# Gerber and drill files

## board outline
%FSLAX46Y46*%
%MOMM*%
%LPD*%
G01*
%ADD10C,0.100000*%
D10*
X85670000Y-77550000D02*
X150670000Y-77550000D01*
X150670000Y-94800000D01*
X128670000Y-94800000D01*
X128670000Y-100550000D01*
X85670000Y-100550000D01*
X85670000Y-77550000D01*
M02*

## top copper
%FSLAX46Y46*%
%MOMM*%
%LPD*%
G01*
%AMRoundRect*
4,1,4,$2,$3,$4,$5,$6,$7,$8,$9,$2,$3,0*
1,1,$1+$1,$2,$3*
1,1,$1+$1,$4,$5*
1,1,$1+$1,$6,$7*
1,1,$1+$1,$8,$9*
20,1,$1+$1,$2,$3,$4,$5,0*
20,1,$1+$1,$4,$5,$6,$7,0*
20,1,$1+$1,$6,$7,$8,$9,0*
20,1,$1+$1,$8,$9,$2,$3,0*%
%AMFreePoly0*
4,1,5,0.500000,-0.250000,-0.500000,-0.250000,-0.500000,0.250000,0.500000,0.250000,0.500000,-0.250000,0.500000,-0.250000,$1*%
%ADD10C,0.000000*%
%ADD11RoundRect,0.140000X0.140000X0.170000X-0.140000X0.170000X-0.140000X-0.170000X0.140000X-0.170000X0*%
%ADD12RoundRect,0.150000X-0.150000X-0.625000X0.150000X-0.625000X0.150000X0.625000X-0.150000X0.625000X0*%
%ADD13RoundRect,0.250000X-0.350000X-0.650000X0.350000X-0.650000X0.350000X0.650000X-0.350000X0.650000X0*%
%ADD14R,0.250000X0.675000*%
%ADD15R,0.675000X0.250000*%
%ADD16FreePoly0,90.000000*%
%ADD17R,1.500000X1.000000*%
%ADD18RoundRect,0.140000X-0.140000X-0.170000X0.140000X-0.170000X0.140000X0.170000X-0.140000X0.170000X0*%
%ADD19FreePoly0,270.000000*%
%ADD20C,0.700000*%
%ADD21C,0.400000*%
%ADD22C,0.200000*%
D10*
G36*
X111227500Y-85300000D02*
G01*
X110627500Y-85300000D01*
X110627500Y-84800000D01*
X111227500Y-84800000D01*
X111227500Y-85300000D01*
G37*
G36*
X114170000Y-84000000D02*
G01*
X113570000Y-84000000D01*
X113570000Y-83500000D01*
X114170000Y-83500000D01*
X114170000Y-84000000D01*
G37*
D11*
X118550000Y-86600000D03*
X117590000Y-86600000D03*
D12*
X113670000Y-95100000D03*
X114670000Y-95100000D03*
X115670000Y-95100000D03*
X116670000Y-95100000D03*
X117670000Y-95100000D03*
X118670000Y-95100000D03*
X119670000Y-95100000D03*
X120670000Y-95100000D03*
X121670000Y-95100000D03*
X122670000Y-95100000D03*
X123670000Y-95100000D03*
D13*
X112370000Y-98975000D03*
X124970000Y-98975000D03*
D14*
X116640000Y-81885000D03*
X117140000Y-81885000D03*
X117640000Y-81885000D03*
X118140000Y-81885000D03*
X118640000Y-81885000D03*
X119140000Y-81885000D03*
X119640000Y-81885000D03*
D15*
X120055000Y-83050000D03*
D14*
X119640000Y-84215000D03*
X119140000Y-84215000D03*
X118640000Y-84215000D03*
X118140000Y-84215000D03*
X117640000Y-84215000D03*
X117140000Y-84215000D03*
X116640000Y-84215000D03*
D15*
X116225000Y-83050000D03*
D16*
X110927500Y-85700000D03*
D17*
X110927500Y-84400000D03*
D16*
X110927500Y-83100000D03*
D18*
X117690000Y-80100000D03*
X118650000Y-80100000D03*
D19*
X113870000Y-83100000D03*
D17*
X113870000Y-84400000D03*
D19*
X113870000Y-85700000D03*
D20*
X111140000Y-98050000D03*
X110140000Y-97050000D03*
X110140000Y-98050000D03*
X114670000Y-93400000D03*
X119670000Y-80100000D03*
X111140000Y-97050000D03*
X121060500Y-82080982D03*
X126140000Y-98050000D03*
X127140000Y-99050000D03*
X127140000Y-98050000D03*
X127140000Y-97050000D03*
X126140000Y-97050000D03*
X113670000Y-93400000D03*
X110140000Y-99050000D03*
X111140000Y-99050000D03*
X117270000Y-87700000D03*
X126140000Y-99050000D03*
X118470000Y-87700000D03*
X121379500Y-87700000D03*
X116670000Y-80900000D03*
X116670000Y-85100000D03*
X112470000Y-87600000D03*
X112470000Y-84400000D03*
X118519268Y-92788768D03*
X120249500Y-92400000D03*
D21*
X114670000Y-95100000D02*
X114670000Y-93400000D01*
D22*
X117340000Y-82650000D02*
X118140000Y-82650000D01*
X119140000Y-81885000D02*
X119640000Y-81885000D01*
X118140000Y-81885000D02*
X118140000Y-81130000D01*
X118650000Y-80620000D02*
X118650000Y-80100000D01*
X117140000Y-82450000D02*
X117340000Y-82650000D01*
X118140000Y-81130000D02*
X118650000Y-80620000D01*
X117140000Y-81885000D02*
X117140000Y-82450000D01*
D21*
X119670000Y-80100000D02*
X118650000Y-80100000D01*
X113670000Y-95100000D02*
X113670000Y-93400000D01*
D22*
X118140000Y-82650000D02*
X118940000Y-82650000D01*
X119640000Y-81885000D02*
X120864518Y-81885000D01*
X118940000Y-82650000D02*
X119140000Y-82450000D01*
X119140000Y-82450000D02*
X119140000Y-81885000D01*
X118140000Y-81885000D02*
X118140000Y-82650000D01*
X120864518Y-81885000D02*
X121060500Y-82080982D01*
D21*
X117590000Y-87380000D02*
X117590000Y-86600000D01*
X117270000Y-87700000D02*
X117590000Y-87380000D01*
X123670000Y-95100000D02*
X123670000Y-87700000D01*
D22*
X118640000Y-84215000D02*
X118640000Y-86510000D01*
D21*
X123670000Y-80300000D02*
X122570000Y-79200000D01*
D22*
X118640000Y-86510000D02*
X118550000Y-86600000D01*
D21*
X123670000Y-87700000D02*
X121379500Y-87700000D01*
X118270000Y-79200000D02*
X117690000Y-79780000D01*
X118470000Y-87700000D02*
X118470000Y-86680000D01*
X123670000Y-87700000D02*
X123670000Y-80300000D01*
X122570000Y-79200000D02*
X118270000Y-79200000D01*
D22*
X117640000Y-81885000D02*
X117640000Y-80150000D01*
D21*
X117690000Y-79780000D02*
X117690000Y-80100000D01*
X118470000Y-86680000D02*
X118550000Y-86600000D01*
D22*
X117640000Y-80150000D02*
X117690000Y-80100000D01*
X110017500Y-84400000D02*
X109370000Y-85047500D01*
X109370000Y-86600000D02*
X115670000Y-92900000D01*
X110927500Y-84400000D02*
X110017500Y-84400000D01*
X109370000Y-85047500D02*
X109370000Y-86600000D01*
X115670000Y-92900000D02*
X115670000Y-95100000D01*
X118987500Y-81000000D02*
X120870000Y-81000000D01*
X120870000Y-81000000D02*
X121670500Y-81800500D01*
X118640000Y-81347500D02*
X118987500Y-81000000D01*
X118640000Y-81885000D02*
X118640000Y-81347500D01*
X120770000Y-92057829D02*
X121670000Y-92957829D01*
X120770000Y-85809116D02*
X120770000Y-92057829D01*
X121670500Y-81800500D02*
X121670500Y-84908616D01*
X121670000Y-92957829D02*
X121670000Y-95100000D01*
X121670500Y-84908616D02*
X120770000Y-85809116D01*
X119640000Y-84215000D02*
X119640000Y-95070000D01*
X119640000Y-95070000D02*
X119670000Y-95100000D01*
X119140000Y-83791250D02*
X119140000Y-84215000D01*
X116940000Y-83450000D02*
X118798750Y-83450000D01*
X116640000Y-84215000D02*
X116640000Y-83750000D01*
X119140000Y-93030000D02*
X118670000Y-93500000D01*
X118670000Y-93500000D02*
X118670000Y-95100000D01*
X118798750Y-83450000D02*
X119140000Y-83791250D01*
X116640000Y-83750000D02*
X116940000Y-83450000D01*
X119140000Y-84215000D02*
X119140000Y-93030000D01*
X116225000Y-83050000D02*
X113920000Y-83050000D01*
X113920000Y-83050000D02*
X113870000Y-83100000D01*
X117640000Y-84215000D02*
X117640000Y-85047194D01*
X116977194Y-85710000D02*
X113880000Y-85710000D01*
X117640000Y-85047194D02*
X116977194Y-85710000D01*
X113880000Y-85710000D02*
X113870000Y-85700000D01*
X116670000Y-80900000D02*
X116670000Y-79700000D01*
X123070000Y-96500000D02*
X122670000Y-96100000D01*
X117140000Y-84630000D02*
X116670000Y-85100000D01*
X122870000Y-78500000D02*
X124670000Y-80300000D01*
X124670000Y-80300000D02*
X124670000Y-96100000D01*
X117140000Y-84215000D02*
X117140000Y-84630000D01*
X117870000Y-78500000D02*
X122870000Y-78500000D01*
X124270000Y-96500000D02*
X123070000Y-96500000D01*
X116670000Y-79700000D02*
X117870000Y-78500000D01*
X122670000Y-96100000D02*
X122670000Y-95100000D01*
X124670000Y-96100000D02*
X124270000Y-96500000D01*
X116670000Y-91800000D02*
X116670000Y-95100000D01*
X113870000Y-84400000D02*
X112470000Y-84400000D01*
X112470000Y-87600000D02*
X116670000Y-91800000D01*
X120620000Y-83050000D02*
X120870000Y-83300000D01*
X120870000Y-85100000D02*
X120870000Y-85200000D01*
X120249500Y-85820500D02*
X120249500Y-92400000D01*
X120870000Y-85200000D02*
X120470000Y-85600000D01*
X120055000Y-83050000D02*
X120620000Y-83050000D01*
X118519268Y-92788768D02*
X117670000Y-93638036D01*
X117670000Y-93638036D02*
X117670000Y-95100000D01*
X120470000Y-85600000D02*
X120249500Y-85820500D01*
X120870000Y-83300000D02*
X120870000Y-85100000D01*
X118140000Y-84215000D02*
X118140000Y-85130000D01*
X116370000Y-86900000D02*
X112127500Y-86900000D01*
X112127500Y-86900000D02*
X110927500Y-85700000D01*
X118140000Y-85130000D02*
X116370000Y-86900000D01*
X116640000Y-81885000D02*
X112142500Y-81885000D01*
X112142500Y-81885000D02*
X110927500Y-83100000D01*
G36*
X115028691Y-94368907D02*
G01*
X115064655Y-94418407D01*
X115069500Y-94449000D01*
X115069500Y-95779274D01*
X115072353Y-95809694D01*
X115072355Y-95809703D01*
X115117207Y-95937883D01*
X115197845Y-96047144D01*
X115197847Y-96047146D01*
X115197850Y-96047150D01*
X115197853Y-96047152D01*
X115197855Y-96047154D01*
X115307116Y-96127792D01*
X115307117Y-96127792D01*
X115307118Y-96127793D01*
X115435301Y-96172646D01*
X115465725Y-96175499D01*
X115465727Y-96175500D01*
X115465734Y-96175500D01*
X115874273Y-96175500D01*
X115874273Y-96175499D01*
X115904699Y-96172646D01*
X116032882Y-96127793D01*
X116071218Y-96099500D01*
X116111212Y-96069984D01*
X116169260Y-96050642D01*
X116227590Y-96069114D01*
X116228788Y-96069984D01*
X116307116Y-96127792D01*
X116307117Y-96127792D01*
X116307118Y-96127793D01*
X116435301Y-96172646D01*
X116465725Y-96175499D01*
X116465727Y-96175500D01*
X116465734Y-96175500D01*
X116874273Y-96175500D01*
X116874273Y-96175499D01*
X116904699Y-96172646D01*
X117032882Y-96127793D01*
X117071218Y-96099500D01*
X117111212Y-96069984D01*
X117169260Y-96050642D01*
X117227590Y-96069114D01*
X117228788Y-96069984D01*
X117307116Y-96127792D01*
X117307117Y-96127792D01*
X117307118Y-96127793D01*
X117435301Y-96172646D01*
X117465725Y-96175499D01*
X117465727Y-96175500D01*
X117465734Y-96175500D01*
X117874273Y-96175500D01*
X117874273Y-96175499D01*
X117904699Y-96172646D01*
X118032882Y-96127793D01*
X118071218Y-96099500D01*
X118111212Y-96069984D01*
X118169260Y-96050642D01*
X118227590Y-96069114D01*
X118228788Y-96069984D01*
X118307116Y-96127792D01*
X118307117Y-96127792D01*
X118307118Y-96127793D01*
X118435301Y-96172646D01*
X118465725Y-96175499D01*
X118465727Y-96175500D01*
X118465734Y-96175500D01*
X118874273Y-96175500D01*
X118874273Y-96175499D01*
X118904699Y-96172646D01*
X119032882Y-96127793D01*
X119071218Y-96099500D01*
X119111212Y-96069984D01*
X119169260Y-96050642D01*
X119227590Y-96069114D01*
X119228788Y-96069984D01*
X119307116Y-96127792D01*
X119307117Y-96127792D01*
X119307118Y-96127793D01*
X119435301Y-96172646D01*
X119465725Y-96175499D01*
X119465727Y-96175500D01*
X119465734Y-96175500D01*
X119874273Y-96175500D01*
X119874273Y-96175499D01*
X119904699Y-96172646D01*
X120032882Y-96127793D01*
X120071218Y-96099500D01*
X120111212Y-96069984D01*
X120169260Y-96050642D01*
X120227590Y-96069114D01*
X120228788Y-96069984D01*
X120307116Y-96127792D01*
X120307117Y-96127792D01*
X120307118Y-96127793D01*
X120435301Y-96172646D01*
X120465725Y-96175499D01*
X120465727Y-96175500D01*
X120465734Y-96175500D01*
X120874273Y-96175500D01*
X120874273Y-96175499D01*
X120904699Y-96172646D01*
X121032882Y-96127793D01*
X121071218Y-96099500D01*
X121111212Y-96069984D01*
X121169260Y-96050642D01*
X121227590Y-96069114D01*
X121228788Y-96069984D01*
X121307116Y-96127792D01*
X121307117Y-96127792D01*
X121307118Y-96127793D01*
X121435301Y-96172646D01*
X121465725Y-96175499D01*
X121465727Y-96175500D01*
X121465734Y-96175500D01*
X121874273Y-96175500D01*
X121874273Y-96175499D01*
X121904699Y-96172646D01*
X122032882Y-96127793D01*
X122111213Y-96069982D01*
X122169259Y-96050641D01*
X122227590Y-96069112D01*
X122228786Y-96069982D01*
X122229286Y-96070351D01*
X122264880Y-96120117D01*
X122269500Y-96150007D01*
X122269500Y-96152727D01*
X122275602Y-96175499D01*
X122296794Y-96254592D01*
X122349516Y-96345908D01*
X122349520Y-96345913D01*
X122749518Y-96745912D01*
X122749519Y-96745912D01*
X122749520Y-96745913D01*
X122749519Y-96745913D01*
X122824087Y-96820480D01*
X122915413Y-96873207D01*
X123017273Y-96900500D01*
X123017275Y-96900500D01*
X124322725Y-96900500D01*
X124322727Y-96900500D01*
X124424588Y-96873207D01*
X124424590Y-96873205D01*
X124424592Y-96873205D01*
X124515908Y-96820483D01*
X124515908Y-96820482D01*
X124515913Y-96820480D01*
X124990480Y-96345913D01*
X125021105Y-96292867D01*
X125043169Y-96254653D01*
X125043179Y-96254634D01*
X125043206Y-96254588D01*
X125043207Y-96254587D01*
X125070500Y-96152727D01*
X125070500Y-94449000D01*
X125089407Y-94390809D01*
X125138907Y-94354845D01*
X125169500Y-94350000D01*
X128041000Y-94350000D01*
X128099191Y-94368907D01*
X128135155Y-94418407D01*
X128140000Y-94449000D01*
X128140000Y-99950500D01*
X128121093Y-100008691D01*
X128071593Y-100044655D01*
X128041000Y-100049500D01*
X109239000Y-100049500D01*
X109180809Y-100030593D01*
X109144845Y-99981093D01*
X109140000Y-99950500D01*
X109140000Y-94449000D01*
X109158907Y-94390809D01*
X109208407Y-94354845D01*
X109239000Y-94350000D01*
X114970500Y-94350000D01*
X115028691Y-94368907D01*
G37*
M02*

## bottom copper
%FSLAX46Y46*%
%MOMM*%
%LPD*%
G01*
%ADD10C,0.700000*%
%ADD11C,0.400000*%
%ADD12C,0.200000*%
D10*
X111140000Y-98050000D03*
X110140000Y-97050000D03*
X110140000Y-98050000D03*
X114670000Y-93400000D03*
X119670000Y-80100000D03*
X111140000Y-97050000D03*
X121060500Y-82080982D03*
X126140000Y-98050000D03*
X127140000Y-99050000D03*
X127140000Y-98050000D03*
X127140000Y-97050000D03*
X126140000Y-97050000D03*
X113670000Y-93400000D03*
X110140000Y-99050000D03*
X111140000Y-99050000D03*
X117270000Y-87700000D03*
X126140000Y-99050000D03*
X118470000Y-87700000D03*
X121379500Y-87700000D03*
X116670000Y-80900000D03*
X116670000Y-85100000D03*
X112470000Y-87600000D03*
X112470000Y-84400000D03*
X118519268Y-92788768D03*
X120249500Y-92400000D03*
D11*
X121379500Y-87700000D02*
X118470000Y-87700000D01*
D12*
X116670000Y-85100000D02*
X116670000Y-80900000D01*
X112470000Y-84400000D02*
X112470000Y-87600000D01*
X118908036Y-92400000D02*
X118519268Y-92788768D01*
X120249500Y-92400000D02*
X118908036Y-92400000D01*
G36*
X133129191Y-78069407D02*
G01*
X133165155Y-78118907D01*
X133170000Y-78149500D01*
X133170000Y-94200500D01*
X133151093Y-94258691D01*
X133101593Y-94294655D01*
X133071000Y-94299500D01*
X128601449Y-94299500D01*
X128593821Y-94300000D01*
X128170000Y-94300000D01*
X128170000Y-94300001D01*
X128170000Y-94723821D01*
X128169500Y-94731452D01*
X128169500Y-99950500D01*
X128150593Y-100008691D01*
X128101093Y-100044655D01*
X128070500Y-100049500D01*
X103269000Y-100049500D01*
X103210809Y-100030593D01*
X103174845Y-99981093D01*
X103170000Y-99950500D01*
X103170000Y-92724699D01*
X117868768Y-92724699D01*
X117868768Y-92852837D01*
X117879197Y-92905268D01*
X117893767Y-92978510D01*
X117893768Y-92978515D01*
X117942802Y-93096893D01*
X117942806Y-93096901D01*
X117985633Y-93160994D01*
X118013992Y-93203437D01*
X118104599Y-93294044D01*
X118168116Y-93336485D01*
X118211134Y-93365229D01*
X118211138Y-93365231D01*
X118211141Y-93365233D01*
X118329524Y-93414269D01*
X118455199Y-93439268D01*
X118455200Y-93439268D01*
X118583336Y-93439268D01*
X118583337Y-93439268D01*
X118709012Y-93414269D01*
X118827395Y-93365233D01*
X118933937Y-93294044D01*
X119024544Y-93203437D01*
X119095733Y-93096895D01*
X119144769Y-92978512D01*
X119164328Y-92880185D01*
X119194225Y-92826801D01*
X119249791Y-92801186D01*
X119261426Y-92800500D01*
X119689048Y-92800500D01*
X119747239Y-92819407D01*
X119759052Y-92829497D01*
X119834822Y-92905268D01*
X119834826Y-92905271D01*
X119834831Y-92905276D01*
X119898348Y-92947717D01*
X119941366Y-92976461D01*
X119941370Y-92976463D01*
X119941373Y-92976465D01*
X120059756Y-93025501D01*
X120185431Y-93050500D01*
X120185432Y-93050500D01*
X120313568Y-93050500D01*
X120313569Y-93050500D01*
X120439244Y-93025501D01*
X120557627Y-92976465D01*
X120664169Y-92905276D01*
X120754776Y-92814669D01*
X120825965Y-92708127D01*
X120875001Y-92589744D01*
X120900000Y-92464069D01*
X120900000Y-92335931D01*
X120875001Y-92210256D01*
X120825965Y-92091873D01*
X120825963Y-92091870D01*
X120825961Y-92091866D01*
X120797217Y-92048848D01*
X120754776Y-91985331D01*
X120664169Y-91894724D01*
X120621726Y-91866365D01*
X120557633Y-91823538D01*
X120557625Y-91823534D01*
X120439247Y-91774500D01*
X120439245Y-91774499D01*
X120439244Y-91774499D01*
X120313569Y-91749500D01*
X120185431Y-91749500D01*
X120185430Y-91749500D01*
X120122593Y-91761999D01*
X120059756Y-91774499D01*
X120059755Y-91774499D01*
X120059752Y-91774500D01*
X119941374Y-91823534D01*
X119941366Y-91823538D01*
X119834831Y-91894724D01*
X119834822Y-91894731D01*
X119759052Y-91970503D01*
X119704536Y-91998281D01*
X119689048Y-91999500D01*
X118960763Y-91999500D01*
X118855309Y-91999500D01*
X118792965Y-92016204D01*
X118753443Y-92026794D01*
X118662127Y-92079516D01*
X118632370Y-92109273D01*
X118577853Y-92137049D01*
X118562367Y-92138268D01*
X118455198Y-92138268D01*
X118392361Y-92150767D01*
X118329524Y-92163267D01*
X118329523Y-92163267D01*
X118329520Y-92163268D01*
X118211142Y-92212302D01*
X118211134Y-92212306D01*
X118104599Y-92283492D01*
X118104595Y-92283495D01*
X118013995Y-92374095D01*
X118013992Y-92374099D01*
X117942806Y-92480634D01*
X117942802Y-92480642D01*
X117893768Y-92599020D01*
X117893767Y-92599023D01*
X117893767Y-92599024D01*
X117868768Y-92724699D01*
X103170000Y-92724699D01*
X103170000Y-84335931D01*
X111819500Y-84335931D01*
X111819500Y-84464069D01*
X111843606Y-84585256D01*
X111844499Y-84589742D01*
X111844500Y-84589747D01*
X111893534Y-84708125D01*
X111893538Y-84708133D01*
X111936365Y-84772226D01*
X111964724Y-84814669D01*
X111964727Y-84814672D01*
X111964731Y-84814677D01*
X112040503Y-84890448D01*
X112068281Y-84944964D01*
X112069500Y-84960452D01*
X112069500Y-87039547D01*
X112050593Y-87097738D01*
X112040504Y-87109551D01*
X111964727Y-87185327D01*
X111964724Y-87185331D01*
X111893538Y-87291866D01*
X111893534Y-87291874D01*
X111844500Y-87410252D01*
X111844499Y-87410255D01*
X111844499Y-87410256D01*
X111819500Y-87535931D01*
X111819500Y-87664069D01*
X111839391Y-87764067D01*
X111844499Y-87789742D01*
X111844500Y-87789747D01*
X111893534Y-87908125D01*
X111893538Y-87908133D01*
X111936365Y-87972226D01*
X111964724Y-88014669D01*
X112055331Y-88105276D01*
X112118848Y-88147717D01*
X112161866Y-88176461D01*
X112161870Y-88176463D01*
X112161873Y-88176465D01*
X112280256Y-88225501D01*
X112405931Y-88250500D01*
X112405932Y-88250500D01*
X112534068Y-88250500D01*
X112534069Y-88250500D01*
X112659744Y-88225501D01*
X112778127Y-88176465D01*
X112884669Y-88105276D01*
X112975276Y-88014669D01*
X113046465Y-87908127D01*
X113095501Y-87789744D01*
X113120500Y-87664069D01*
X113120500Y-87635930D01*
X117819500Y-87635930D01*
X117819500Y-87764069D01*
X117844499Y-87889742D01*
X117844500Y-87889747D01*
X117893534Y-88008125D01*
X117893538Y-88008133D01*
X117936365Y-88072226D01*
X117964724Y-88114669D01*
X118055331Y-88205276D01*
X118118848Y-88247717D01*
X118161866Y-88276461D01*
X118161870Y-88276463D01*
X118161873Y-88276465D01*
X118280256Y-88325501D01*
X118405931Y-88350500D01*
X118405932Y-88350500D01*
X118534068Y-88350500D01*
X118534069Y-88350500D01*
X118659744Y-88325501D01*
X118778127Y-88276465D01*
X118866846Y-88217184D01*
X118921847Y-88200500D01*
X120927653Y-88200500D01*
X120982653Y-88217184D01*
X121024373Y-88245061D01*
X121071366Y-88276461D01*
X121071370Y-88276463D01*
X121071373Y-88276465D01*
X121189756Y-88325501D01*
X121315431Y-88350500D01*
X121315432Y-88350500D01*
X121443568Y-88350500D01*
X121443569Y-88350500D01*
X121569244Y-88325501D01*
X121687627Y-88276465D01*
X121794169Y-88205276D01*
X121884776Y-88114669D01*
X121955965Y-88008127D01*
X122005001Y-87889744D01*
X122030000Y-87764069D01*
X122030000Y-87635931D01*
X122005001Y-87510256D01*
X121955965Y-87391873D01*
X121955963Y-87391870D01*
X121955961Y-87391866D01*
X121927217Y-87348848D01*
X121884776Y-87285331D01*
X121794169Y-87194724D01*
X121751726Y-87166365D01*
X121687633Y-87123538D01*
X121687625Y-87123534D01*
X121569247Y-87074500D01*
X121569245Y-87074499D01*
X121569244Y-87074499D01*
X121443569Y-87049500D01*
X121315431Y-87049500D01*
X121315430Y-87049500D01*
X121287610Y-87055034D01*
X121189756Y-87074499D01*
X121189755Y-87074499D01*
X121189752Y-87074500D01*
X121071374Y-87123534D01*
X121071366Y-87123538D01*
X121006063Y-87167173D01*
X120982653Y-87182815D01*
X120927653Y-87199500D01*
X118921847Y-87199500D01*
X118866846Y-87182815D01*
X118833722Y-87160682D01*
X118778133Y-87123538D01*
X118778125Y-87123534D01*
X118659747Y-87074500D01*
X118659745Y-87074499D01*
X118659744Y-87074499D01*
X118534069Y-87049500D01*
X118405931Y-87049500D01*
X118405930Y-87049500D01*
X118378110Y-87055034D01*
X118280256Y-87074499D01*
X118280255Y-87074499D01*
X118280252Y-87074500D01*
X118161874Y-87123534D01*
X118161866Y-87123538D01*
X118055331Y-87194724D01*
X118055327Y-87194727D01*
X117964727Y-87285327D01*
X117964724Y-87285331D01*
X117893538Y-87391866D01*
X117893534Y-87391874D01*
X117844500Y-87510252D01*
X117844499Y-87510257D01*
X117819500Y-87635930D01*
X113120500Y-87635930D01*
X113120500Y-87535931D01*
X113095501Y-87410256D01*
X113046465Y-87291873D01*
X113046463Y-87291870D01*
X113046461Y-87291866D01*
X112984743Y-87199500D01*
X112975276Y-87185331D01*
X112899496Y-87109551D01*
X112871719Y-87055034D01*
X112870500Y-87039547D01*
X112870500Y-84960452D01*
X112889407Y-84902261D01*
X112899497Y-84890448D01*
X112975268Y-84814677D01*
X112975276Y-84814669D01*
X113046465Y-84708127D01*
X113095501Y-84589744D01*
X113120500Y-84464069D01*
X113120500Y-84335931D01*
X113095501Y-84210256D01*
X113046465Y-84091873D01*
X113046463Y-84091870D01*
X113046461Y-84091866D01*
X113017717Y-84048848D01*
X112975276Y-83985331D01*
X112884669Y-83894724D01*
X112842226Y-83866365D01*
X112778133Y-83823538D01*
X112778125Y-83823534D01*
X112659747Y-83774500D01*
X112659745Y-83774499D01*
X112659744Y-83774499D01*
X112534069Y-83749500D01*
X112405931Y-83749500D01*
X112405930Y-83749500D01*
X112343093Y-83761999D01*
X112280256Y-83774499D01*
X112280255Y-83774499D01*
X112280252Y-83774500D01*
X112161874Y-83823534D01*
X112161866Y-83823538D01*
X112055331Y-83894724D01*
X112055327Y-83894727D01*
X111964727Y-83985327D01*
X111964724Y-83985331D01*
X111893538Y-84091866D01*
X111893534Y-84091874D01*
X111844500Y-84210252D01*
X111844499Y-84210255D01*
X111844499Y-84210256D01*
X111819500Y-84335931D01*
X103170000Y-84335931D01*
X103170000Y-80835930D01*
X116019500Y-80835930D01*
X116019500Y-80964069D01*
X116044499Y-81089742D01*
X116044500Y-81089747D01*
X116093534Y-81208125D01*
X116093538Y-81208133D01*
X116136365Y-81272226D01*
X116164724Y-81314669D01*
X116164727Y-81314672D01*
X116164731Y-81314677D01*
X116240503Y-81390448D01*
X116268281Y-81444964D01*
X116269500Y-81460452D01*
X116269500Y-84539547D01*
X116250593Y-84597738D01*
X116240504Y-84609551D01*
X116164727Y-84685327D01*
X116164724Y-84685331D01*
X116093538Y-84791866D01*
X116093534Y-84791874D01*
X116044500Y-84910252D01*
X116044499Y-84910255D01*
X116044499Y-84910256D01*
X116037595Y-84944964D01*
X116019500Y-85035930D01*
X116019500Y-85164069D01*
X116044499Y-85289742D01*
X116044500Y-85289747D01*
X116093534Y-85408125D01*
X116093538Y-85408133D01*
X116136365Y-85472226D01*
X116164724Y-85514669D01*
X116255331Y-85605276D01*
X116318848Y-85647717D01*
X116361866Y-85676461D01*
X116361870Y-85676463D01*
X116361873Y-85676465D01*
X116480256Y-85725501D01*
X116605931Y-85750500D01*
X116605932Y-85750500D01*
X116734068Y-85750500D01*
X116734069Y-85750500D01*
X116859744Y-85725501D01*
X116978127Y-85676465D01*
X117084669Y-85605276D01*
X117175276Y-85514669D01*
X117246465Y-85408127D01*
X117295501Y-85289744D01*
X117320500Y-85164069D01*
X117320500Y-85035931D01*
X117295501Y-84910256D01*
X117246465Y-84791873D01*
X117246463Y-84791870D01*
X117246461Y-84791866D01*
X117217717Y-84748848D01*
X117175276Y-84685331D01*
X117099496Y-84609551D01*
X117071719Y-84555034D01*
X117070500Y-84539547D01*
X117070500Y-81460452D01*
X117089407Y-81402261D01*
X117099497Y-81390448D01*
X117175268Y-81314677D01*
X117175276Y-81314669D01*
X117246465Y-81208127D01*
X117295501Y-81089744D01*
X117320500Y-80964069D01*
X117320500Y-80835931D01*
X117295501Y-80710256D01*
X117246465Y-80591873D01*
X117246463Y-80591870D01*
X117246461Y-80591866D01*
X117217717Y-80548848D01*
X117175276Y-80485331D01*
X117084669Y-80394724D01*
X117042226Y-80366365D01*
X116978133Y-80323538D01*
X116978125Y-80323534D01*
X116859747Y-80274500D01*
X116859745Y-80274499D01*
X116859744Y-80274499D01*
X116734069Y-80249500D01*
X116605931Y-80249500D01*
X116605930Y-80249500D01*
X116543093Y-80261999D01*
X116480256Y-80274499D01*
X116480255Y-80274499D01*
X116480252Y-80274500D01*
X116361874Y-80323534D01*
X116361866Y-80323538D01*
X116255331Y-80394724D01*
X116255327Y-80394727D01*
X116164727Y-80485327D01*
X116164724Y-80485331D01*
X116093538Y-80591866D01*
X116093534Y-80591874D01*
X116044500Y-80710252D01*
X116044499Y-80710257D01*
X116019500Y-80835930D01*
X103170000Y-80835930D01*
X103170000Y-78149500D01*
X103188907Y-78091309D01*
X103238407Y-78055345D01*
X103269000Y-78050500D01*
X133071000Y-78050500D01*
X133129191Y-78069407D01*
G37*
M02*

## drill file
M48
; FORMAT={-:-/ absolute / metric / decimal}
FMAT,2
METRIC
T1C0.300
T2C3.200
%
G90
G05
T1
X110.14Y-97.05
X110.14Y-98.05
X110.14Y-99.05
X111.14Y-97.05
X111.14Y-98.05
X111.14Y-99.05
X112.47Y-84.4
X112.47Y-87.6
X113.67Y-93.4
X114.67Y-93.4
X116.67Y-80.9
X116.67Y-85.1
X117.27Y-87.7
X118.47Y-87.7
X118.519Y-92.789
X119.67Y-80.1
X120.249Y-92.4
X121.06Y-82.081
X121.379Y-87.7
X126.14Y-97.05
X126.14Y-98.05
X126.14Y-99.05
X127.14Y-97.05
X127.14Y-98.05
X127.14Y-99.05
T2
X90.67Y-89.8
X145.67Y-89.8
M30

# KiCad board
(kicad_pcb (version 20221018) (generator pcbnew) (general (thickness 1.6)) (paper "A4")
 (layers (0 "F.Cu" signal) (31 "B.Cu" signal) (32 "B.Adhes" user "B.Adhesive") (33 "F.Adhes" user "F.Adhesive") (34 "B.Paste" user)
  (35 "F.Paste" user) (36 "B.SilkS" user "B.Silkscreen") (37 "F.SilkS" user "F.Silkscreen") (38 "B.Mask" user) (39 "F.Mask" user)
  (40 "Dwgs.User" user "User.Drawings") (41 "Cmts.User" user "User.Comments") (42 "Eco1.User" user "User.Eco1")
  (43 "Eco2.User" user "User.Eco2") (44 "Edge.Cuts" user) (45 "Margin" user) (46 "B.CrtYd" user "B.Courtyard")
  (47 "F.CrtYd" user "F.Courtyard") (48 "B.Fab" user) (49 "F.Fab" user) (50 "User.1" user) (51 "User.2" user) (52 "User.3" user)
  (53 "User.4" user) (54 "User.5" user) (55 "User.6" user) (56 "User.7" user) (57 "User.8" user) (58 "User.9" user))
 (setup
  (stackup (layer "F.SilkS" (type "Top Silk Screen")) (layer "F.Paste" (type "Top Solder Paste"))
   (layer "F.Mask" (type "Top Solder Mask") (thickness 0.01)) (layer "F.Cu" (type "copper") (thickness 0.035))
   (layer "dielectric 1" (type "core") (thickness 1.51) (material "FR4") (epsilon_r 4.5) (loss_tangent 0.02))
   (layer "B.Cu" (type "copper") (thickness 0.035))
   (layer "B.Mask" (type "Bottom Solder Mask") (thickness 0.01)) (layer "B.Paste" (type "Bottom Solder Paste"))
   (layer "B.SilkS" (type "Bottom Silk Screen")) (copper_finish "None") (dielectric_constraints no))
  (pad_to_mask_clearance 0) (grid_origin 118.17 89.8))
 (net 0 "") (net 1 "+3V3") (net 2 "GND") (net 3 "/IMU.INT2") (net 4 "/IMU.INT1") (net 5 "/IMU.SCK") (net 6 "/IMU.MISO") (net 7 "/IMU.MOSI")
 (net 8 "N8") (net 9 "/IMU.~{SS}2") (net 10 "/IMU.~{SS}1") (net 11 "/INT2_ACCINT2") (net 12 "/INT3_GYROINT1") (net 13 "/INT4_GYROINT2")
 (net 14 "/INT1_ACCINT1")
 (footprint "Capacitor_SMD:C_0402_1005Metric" (layer "F.Cu") (at 118.07 86.6 180)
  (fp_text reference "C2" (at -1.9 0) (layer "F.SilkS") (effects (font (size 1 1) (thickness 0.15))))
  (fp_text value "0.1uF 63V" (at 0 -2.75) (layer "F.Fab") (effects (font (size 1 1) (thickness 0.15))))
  (pad "1" smd roundrect (at -0.48 0 180) (size 0.56 0.62) (layers "F.Cu" "F.Paste" "F.Mask") (roundrect_rratio 0.25) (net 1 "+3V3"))
  (pad "2" smd roundrect (at 0.48 0 180) (size 0.56 0.62) (layers "F.Cu" "F.Paste" "F.Mask") (roundrect_rratio 0.25) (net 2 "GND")))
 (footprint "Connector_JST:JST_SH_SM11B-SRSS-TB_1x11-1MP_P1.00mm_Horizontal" (layer "F.Cu") (at 118.67 97.1)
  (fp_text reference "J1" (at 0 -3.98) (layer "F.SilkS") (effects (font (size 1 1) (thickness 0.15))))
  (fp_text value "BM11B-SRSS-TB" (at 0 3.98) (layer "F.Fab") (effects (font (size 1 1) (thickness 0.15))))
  (pad "1" smd roundrect (at -5 -2) (size 0.6 1.55) (layers "F.Cu" "F.Paste" "F.Mask") (roundrect_rratio 0.25) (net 2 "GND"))
  (pad "2" smd roundrect (at -4 -2) (size 0.6 1.55) (layers "F.Cu" "F.Paste" "F.Mask") (roundrect_rratio 0.25) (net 2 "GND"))
  (pad "3" smd roundrect (at -3 -2) (size 0.6 1.55) (layers "F.Cu" "F.Paste" "F.Mask") (roundrect_rratio 0.25) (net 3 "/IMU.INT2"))
  (pad "4" smd roundrect (at -2 -2) (size 0.6 1.55) (layers "F.Cu" "F.Paste" "F.Mask") (roundrect_rratio 0.25) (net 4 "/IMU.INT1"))
  (pad "5" smd roundrect (at -1 -2) (size 0.6 1.55) (layers "F.Cu" "F.Paste" "F.Mask") (roundrect_rratio 0.25) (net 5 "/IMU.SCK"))
  (pad "6" smd roundrect (at 0 -2) (size 0.6 1.55) (layers "F.Cu" "F.Paste" "F.Mask") (roundrect_rratio 0.25) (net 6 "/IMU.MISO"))
  (pad "7" smd roundrect (at 1 -2) (size 0.6 1.55) (layers "F.Cu" "F.Paste" "F.Mask") (roundrect_rratio 0.25) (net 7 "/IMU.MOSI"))
  (pad "8" smd roundrect (at 2 -2) (size 0.6 1.55) (layers "F.Cu" "F.Paste" "F.Mask") (roundrect_rratio 0.25) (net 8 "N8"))
  (pad "9" smd roundrect (at 3 -2) (size 0.6 1.55) (layers "F.Cu" "F.Paste" "F.Mask") (roundrect_rratio 0.25) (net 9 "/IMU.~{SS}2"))
  (pad "10" smd roundrect (at 4 -2) (size 0.6 1.55) (layers "F.Cu" "F.Paste" "F.Mask") (roundrect_rratio 0.25) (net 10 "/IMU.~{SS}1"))
  (pad "11" smd roundrect (at 5 -2) (size 0.6 1.55) (layers "F.Cu" "F.Paste" "F.Mask") (roundrect_rratio 0.25) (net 1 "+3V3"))
  (pad "MP" smd roundrect (at -6.3 1.875) (size 1.2 1.8) (layers "F.Cu" "F.Paste" "F.Mask") (roundrect_rratio 0.2083333333) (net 2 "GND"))
  (pad "MP" smd roundrect (at 6.3 1.875) (size 1.2 1.8) (layers "F.Cu" "F.Paste" "F.Mask") (roundrect_rratio 0.2083333333) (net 2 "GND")))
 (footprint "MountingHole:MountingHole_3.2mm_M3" (layer "F.Cu") (at 90.67 89.8)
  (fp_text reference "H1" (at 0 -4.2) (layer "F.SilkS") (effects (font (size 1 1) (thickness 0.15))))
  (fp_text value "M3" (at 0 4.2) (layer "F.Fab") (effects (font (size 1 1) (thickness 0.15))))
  (pad "" np_thru_hole circle (at 0 0) (size 3.2 3.2) (drill 3.2) (layers "*.Cu" "*.Mask")))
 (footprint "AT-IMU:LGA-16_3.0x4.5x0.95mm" (layer "F.Cu") (at 118.14 83.05)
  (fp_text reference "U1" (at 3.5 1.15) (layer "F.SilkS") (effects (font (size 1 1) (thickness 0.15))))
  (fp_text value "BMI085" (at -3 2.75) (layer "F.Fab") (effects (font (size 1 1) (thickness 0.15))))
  (pad "1" smd rect (at -1.5 -1.165) (size 0.25 0.675) (layers "F.Cu" "F.Paste" "F.Mask") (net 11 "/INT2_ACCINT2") (solder_mask_margin 0.05))
  (pad "2" smd rect (at -1 -1.165) (size 0.25 0.675) (layers "F.Cu" "F.Paste" "F.Mask") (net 2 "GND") (solder_mask_margin 0.05))
  (pad "3" smd rect (at -0.5 -1.165) (size 0.25 0.675) (layers "F.Cu" "F.Paste" "F.Mask") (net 1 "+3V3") (solder_mask_margin 0.05))
  (pad "4" smd rect (at 0 -1.165) (size 0.25 0.675) (layers "F.Cu" "F.Paste" "F.Mask") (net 2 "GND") (solder_mask_margin 0.05))
  (pad "5" smd rect (at 0.5 -1.165) (size 0.25 0.675) (layers "F.Cu" "F.Paste" "F.Mask") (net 9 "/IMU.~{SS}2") (solder_mask_margin 0.05))
  (pad "6" smd rect (at 1 -1.165) (size 0.25 0.675) (layers "F.Cu" "F.Paste" "F.Mask") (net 2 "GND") (solder_mask_margin 0.05))
  (pad "7" smd rect (at 1.5 -1.165) (size 0.25 0.675) (layers "F.Cu" "F.Paste" "F.Mask") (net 2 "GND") (solder_mask_margin 0.05))
  (pad "8" smd rect (at 1.915 0 270) (size 0.25 0.675) (layers "F.Cu" "F.Paste" "F.Mask") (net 5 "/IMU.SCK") (solder_mask_margin 0.05))
  (pad "9" smd rect (at 1.5 1.165) (size 0.25 0.675) (layers "F.Cu" "F.Paste" "F.Mask") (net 7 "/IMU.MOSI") (solder_mask_margin 0.05))
  (pad "10" smd rect (at 1 1.165) (size 0.25 0.675) (layers "F.Cu" "F.Paste" "F.Mask") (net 6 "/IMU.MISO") (solder_mask_margin 0.05))
  (pad "11" smd rect (at 0.5 1.165) (size 0.25 0.675) (layers "F.Cu" "F.Paste" "F.Mask") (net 1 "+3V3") (solder_mask_margin 0.05))
  (pad "12" smd rect (at 0 1.165) (size 0.25 0.675) (layers "F.Cu" "F.Paste" "F.Mask") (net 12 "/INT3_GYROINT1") (solder_mask_margin 0.05))
  (pad "13" smd rect (at -0.5 1.165) (size 0.25 0.675) (layers "F.Cu" "F.Paste" "F.Mask") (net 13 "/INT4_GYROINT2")
   (solder_mask_margin 0.05))
  (pad "14" smd rect (at -1 1.165) (size 0.25 0.675) (layers "F.Cu" "F.Paste" "F.Mask") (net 10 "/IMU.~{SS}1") (solder_mask_margin 0.05))
  (pad "15" smd rect (at -1.5 1.165) (size 0.25 0.675) (layers "F.Cu" "F.Paste" "F.Mask") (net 6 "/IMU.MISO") (solder_mask_margin 0.05))
  (pad "16" smd rect (at -1.915 0 90) (size 0.25 0.675) (layers "F.Cu" "F.Paste" "F.Mask") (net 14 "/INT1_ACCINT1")
   (solder_mask_margin 0.05)))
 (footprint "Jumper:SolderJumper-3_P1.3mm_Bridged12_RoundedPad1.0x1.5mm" (layer "F.Cu") (at 110.9275 84.4 90) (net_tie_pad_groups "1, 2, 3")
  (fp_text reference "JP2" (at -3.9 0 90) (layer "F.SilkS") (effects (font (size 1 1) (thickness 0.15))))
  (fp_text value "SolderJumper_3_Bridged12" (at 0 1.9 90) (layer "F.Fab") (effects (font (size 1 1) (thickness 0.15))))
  (fp_poly (pts (xy -0.9 -0.3) (xy -0.4 -0.3) (xy -0.4 0.3) (xy -0.9 0.3)) (stroke (width 0) (type solid)) (fill solid) (layer "F.Cu"))
  (pad "1" smd custom (at -1.3 0 90) (size 1 0.5) (layers "F.Cu" "F.Mask") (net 12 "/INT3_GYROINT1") (zone_connect 2)
   (thermal_bridge_angle 45) (options (clearance outline) (anchor rect)) (primitives))
  (pad "2" smd rect (at 0 0 90) (size 1 1.5) (layers "F.Cu" "F.Mask") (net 3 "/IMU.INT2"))
  (pad "3" smd custom (at 1.3 0 90) (size 1 0.5) (layers "F.Cu" "F.Mask") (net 11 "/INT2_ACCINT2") (zone_connect 2)
   (thermal_bridge_angle 45) (options (clearance outline) (anchor rect)) (primitives)))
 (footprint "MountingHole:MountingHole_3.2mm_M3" (layer "F.Cu") (at 145.67 89.8)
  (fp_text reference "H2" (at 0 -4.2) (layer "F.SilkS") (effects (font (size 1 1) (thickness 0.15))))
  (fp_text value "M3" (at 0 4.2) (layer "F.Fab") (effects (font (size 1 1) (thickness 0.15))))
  (pad "" np_thru_hole circle (at 0 0) (size 3.2 3.2) (drill 3.2) (layers "*.Cu" "*.Mask")))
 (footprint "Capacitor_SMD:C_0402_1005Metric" (layer "F.Cu") (at 118.17 80.1)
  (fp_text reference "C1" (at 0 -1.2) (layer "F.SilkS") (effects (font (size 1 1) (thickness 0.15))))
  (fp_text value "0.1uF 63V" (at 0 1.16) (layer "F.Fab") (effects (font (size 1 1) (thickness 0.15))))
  (pad "1" smd roundrect (at -0.48 0) (size 0.56 0.62) (layers "F.Cu" "F.Paste" "F.Mask") (roundrect_rratio 0.25) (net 1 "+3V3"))
  (pad "2" smd roundrect (at 0.48 0) (size 0.56 0.62) (layers "F.Cu" "F.Paste" "F.Mask") (roundrect_rratio 0.25) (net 2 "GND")))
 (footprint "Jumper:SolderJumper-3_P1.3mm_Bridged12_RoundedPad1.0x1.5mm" (layer "F.Cu") (at 113.87 84.4 -90) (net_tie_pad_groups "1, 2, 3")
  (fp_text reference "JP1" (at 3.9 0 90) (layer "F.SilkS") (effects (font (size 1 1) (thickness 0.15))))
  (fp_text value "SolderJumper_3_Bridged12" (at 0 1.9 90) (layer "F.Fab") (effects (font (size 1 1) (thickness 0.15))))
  (fp_poly (pts (xy -0.9 -0.3) (xy -0.4 -0.3) (xy -0.4 0.3) (xy -0.9 0.3)) (stroke (width 0) (type solid)) (fill solid) (layer "F.Cu"))
  (pad "1" smd custom (at -1.3 0 270) (size 1 0.5) (layers "F.Cu" "F.Mask") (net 14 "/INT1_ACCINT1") (zone_connect 2)
   (thermal_bridge_angle 45) (options (clearance outline) (anchor rect)) (primitives))
  (pad "2" smd rect (at 0 0 270) (size 1 1.5) (layers "F.Cu" "F.Mask") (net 4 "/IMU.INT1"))
  (pad "3" smd custom (at 1.3 0 270) (size 1 0.5) (layers "F.Cu" "F.Mask") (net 13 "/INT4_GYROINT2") (zone_connect 2)
   (thermal_bridge_angle 45) (options (clearance outline) (anchor rect)) (primitives)))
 (gr_poly
  (pts (xy 85.67 77.55) (xy 150.67 77.55) (xy 150.67 94.8) (xy 128.67 94.8) (xy 128.67 100.55) (xy 85.67 100.55))
  (stroke (width 0.1) (type solid)) (fill none) (layer "Edge.Cuts"))
 (segment (start 114.67 95.1) (end 114.67 93.4) (width 0.4) (layer "F.Cu") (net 2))
 (segment (start 117.34 82.65) (end 118.14 82.65) (width 0.2) (layer "F.Cu") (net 2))
 (segment (start 119.14 81.885) (end 119.64 81.885) (width 0.2) (layer "F.Cu") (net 2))
 (segment (start 118.14 81.885) (end 118.14 81.13) (width 0.2) (layer "F.Cu") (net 2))
 (segment (start 118.65 80.62) (end 118.65 80.1) (width 0.2) (layer "F.Cu") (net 2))
 (segment (start 117.14 82.45) (end 117.34 82.65) (width 0.2) (layer "F.Cu") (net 2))
 (segment (start 118.14 81.13) (end 118.65 80.62) (width 0.2) (layer "F.Cu") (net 2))
 (segment (start 117.14 81.885) (end 117.14 82.45) (width 0.2) (layer "F.Cu") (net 2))
 (segment (start 119.67 80.1) (end 118.65 80.1) (width 0.4) (layer "F.Cu") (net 2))
 (segment (start 113.67 95.1) (end 113.67 93.4) (width 0.4) (layer "F.Cu") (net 2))
 (segment (start 118.14 82.65) (end 118.94 82.65) (width 0.2) (layer "F.Cu") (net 2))
 (segment (start 119.64 81.885) (end 120.864518 81.885) (width 0.2) (layer "F.Cu") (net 2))
 (segment (start 118.94 82.65) (end 119.14 82.45) (width 0.2) (layer "F.Cu") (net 2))
 (segment (start 119.14 82.45) (end 119.14 81.885) (width 0.2) (layer "F.Cu") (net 2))
 (segment (start 118.14 81.885) (end 118.14 82.65) (width 0.2) (layer "F.Cu") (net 2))
 (segment (start 120.864518 81.885) (end 121.0605 82.080982) (width 0.2) (layer "F.Cu") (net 2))
 (segment (start 117.59 87.38) (end 117.59 86.6) (width 0.4) (layer "F.Cu") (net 2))
 (segment (start 117.27 87.7) (end 117.59 87.38) (width 0.4) (layer "F.Cu") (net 2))
 (via (at 111.14 98.05) (size 0.7) (drill 0.3) (layers "F.Cu" "B.Cu") (free) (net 2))
 (via (at 110.14 97.05) (size 0.7) (drill 0.3) (layers "F.Cu" "B.Cu") (free) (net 2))
 (via (at 110.14 98.05) (size 0.7) (drill 0.3) (layers "F.Cu" "B.Cu") (free) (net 2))
 (via (at 114.67 93.4) (size 0.7) (drill 0.3) (layers "F.Cu" "B.Cu") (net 2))
 (via (at 119.67 80.1) (size 0.7) (drill 0.3) (layers "F.Cu" "B.Cu") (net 2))
 (via (at 111.14 97.05) (size 0.7) (drill 0.3) (layers "F.Cu" "B.Cu") (free) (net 2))
 (via (at 121.0605 82.080982) (size 0.7) (drill 0.3) (layers "F.Cu" "B.Cu") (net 2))
 (via (at 126.14 98.05) (size 0.7) (drill 0.3) (layers "F.Cu" "B.Cu") (free) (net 2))
 (via (at 127.14 99.05) (size 0.7) (drill 0.3) (layers "F.Cu" "B.Cu") (free) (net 2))
 (via (at 127.14 98.05) (size 0.7) (drill 0.3) (layers "F.Cu" "B.Cu") (free) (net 2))
 (via (at 127.14 97.05) (size 0.7) (drill 0.3) (layers "F.Cu" "B.Cu") (free) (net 2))
 (via (at 126.14 97.05) (size 0.7) (drill 0.3) (layers "F.Cu" "B.Cu") (free) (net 2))
 (via (at 113.67 93.4) (size 0.7) (drill 0.3) (layers "F.Cu" "B.Cu") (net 2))
 (via (at 110.14 99.05) (size 0.7) (drill 0.3) (layers "F.Cu" "B.Cu") (free) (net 2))
 (via (at 111.14 99.05) (size 0.7) (drill 0.3) (layers "F.Cu" "B.Cu") (free) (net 2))
 (via (at 117.27 87.7) (size 0.7) (drill 0.3) (layers "F.Cu" "B.Cu") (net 2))
 (via (at 126.14 99.05) (size 0.7) (drill 0.3) (layers "F.Cu" "B.Cu") (free) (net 2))
 (segment (start 123.67 95.1) (end 123.67 87.7) (width 0.4) (layer "F.Cu") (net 1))
 (segment (start 118.64 84.215) (end 118.64 86.51) (width 0.2) (layer "F.Cu") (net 1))
 (segment (start 123.67 80.3) (end 122.57 79.2) (width 0.4) (layer "F.Cu") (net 1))
 (segment (start 118.64 86.51) (end 118.55 86.6) (width 0.2) (layer "F.Cu") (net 1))
 (segment (start 123.67 87.7) (end 121.3795 87.7) (width 0.4) (layer "F.Cu") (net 1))
 (segment (start 118.27 79.2) (end 117.69 79.78) (width 0.4) (layer "F.Cu") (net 1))
 (segment (start 118.47 87.7) (end 118.47 86.68) (width 0.4) (layer "F.Cu") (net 1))
 (segment (start 123.67 87.7) (end 123.67 80.3) (width 0.4) (layer "F.Cu") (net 1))
 (segment (start 122.57 79.2) (end 118.27 79.2) (width 0.4) (layer "F.Cu") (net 1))
 (segment (start 117.64 81.885) (end 117.64 80.15) (width 0.2) (layer "F.Cu") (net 1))
 (segment (start 117.69 79.78) (end 117.69 80.1) (width 0.4) (layer "F.Cu") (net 1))
 (segment (start 118.47 86.68) (end 118.55 86.6) (width 0.4) (layer "F.Cu") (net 1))
 (segment (start 117.64 80.15) (end 117.69 80.1) (width 0.2) (layer "F.Cu") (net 1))
 (via (at 118.47 87.7) (size 0.7) (drill 0.3) (layers "F.Cu" "B.Cu") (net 1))
 (via (at 121.3795 87.7) (size 0.7) (drill 0.3) (layers "F.Cu" "B.Cu") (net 1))
 (segment (start 121.3795 87.7) (end 118.47 87.7) (width 0.4) (layer "B.Cu") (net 1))
 (segment (start 110.0175 84.4) (end 109.37 85.0475) (width 0.2) (layer "F.Cu") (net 3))
 (segment (start 109.37 86.6) (end 115.67 92.9) (width 0.2) (layer "F.Cu") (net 3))
 (segment (start 110.9275 84.4) (end 110.0175 84.4) (width 0.2) (layer "F.Cu") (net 3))
 (segment (start 109.37 85.0475) (end 109.37 86.6) (width 0.2) (layer "F.Cu") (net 3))
 (segment (start 115.67 92.9) (end 115.67 95.1) (width 0.2) (layer "F.Cu") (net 3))
 (segment (start 118.9875 81) (end 120.87 81) (width 0.2) (layer "F.Cu") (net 9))
 (segment (start 120.87 81) (end 121.6705 81.8005) (width 0.2) (layer "F.Cu") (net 9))
 (segment (start 118.64 81.3475) (end 118.9875 81) (width 0.2) (layer "F.Cu") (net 9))
 (segment (start 118.64 81.885) (end 118.64 81.3475) (width 0.2) (layer "F.Cu") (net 9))
 (segment (start 120.77 92.057829) (end 121.67 92.957829) (width 0.2) (layer "F.Cu") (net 9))
 (segment (start 120.77 85.809116) (end 120.77 92.057829) (width 0.2) (layer "F.Cu") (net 9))
 (segment (start 121.6705 81.8005) (end 121.6705 84.908616) (width 0.2) (layer "F.Cu") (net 9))
 (segment (start 121.67 92.957829) (end 121.67 95.1) (width 0.2) (layer "F.Cu") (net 9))
 (segment (start 121.6705 84.908616) (end 120.77 85.809116) (width 0.2) (layer "F.Cu") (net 9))
 (segment (start 119.64 84.215) (end 119.64 95.07) (width 0.2) (layer "F.Cu") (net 7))
 (segment (start 119.64 95.07) (end 119.67 95.1) (width 0.2) (layer "F.Cu") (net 7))
 (segment (start 119.14 83.79125) (end 119.14 84.215) (width 0.2) (layer "F.Cu") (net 6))
 (segment (start 116.94 83.45) (end 118.79875 83.45) (width 0.2) (layer "F.Cu") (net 6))
 (segment (start 116.64 84.215) (end 116.64 83.75) (width 0.2) (layer "F.Cu") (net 6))
 (segment (start 119.14 93.03) (end 118.67 93.5) (width 0.2) (layer "F.Cu") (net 6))
 (segment (start 118.67 93.5) (end 118.67 95.1) (width 0.2) (layer "F.Cu") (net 6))
 (segment (start 118.79875 83.45) (end 119.14 83.79125) (width 0.2) (layer "F.Cu") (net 6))
 (segment (start 116.64 83.75) (end 116.94 83.45) (width 0.2) (layer "F.Cu") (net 6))
 (segment (start 119.14 84.215) (end 119.14 93.03) (width 0.2) (layer "F.Cu") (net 6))
 (segment (start 116.225 83.05) (end 113.92 83.05) (width 0.2) (layer "F.Cu") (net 14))
 (segment (start 113.92 83.05) (end 113.87 83.1) (width 0.2) (layer "F.Cu") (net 14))
 (segment (start 117.64 84.215) (end 117.64 85.047194) (width 0.2) (layer "F.Cu") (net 13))
 (segment (start 116.977194 85.71) (end 113.88 85.71) (width 0.2) (layer "F.Cu") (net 13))
 (segment (start 117.64 85.047194) (end 116.977194 85.71) (width 0.2) (layer "F.Cu") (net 13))
 (segment (start 113.88 85.71) (end 113.87 85.7) (width 0.2) (layer "F.Cu") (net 13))
 (segment (start 116.67 80.9) (end 116.67 79.7) (width 0.2) (layer "F.Cu") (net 10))
 (segment (start 123.07 96.5) (end 122.67 96.1) (width 0.2) (layer "F.Cu") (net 10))
 (segment (start 117.14 84.63) (end 116.67 85.1) (width 0.2) (layer "F.Cu") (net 10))
 (segment (start 122.87 78.5) (end 124.67 80.3) (width 0.2) (layer "F.Cu") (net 10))
 (segment (start 124.67 80.3) (end 124.67 96.1) (width 0.2) (layer "F.Cu") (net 10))
 (segment (start 117.14 84.215) (end 117.14 84.63) (width 0.2) (layer "F.Cu") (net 10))
 (segment (start 117.87 78.5) (end 122.87 78.5) (width 0.2) (layer "F.Cu") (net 10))
 (segment (start 124.27 96.5) (end 123.07 96.5) (width 0.2) (layer "F.Cu") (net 10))
 (segment (start 116.67 79.7) (end 117.87 78.5) (width 0.2) (layer "F.Cu") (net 10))
 (segment (start 122.67 96.1) (end 122.67 95.1) (width 0.2) (layer "F.Cu") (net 10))
 (segment (start 124.67 96.1) (end 124.27 96.5) (width 0.2) (layer "F.Cu") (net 10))
 (via (at 116.67 80.9) (size 0.7) (drill 0.3) (layers "F.Cu" "B.Cu") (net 10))
 (via (at 116.67 85.1) (size 0.7) (drill 0.3) (layers "F.Cu" "B.Cu") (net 10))
 (segment (start 116.67 85.1) (end 116.67 80.9) (width 0.2) (layer "B.Cu") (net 10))
 (segment (start 116.67 91.8) (end 116.67 95.1) (width 0.2) (layer "F.Cu") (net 4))
 (segment (start 113.87 84.4) (end 112.47 84.4) (width 0.2) (layer "F.Cu") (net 4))
 (segment (start 112.47 87.6) (end 116.67 91.8) (width 0.2) (layer "F.Cu") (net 4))
 (via (at 112.47 87.6) (size 0.7) (drill 0.3) (layers "F.Cu" "B.Cu") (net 4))
 (via (at 112.47 84.4) (size 0.7) (drill 0.3) (layers "F.Cu" "B.Cu") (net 4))
 (segment (start 112.47 84.4) (end 112.47 87.6) (width 0.2) (layer "B.Cu") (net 4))
 (segment (start 120.62 83.05) (end 120.87 83.3) (width 0.2) (layer "F.Cu") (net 5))
 (segment (start 120.87 85.1) (end 120.87 85.2) (width 0.2) (layer "F.Cu") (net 5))
 (segment (start 120.2495 85.8205) (end 120.2495 92.4) (width 0.2) (layer "F.Cu") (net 5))
 (segment (start 120.87 85.2) (end 120.47 85.6) (width 0.2) (layer "F.Cu") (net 5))
 (segment (start 120.055 83.05) (end 120.62 83.05) (width 0.2) (layer "F.Cu") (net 5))
 (segment (start 118.519268 92.788768) (end 117.67 93.638036) (width 0.2) (layer "F.Cu") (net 5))
 (segment (start 117.67 93.638036) (end 117.67 95.1) (width 0.2) (layer "F.Cu") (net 5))
 (segment (start 120.47 85.6) (end 120.2495 85.8205) (width 0.2) (layer "F.Cu") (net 5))
 (segment (start 120.87 83.3) (end 120.87 85.1) (width 0.2) (layer "F.Cu") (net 5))
 (via (at 118.519268 92.788768) (size 0.7) (drill 0.3) (layers "F.Cu" "B.Cu") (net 5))
 (via (at 120.2495 92.4) (size 0.7) (drill 0.3) (layers "F.Cu" "B.Cu") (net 5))
 (segment (start 118.908036 92.4) (end 118.519268 92.788768) (width 0.2) (layer "B.Cu") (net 5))
 (segment (start 120.2495 92.4) (end 118.908036 92.4) (width 0.2) (layer "B.Cu") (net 5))
 (segment (start 118.14 84.215) (end 118.14 85.13) (width 0.2) (layer "F.Cu") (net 12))
 (segment (start 116.37 86.9) (end 112.1275 86.9) (width 0.2) (layer "F.Cu") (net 12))
 (segment (start 112.1275 86.9) (end 110.9275 85.7) (width 0.2) (layer "F.Cu") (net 12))
 (segment (start 118.14 85.13) (end 116.37 86.9) (width 0.2) (layer "F.Cu") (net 12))
 (segment (start 116.64 81.885) (end 112.1425 81.885) (width 0.2) (layer "F.Cu") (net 11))
 (segment (start 112.1425 81.885) (end 110.9275 83.1) (width 0.2) (layer "F.Cu") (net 11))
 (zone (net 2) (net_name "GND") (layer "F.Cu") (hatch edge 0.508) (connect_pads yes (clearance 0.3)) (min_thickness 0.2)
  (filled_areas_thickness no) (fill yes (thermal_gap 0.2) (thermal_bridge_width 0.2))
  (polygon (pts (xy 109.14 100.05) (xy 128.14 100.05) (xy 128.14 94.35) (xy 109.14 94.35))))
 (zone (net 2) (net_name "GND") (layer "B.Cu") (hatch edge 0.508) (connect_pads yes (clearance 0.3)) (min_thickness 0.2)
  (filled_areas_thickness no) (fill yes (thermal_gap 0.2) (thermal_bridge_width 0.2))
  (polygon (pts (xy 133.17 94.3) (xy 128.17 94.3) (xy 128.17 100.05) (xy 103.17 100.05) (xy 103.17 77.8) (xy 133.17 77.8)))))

